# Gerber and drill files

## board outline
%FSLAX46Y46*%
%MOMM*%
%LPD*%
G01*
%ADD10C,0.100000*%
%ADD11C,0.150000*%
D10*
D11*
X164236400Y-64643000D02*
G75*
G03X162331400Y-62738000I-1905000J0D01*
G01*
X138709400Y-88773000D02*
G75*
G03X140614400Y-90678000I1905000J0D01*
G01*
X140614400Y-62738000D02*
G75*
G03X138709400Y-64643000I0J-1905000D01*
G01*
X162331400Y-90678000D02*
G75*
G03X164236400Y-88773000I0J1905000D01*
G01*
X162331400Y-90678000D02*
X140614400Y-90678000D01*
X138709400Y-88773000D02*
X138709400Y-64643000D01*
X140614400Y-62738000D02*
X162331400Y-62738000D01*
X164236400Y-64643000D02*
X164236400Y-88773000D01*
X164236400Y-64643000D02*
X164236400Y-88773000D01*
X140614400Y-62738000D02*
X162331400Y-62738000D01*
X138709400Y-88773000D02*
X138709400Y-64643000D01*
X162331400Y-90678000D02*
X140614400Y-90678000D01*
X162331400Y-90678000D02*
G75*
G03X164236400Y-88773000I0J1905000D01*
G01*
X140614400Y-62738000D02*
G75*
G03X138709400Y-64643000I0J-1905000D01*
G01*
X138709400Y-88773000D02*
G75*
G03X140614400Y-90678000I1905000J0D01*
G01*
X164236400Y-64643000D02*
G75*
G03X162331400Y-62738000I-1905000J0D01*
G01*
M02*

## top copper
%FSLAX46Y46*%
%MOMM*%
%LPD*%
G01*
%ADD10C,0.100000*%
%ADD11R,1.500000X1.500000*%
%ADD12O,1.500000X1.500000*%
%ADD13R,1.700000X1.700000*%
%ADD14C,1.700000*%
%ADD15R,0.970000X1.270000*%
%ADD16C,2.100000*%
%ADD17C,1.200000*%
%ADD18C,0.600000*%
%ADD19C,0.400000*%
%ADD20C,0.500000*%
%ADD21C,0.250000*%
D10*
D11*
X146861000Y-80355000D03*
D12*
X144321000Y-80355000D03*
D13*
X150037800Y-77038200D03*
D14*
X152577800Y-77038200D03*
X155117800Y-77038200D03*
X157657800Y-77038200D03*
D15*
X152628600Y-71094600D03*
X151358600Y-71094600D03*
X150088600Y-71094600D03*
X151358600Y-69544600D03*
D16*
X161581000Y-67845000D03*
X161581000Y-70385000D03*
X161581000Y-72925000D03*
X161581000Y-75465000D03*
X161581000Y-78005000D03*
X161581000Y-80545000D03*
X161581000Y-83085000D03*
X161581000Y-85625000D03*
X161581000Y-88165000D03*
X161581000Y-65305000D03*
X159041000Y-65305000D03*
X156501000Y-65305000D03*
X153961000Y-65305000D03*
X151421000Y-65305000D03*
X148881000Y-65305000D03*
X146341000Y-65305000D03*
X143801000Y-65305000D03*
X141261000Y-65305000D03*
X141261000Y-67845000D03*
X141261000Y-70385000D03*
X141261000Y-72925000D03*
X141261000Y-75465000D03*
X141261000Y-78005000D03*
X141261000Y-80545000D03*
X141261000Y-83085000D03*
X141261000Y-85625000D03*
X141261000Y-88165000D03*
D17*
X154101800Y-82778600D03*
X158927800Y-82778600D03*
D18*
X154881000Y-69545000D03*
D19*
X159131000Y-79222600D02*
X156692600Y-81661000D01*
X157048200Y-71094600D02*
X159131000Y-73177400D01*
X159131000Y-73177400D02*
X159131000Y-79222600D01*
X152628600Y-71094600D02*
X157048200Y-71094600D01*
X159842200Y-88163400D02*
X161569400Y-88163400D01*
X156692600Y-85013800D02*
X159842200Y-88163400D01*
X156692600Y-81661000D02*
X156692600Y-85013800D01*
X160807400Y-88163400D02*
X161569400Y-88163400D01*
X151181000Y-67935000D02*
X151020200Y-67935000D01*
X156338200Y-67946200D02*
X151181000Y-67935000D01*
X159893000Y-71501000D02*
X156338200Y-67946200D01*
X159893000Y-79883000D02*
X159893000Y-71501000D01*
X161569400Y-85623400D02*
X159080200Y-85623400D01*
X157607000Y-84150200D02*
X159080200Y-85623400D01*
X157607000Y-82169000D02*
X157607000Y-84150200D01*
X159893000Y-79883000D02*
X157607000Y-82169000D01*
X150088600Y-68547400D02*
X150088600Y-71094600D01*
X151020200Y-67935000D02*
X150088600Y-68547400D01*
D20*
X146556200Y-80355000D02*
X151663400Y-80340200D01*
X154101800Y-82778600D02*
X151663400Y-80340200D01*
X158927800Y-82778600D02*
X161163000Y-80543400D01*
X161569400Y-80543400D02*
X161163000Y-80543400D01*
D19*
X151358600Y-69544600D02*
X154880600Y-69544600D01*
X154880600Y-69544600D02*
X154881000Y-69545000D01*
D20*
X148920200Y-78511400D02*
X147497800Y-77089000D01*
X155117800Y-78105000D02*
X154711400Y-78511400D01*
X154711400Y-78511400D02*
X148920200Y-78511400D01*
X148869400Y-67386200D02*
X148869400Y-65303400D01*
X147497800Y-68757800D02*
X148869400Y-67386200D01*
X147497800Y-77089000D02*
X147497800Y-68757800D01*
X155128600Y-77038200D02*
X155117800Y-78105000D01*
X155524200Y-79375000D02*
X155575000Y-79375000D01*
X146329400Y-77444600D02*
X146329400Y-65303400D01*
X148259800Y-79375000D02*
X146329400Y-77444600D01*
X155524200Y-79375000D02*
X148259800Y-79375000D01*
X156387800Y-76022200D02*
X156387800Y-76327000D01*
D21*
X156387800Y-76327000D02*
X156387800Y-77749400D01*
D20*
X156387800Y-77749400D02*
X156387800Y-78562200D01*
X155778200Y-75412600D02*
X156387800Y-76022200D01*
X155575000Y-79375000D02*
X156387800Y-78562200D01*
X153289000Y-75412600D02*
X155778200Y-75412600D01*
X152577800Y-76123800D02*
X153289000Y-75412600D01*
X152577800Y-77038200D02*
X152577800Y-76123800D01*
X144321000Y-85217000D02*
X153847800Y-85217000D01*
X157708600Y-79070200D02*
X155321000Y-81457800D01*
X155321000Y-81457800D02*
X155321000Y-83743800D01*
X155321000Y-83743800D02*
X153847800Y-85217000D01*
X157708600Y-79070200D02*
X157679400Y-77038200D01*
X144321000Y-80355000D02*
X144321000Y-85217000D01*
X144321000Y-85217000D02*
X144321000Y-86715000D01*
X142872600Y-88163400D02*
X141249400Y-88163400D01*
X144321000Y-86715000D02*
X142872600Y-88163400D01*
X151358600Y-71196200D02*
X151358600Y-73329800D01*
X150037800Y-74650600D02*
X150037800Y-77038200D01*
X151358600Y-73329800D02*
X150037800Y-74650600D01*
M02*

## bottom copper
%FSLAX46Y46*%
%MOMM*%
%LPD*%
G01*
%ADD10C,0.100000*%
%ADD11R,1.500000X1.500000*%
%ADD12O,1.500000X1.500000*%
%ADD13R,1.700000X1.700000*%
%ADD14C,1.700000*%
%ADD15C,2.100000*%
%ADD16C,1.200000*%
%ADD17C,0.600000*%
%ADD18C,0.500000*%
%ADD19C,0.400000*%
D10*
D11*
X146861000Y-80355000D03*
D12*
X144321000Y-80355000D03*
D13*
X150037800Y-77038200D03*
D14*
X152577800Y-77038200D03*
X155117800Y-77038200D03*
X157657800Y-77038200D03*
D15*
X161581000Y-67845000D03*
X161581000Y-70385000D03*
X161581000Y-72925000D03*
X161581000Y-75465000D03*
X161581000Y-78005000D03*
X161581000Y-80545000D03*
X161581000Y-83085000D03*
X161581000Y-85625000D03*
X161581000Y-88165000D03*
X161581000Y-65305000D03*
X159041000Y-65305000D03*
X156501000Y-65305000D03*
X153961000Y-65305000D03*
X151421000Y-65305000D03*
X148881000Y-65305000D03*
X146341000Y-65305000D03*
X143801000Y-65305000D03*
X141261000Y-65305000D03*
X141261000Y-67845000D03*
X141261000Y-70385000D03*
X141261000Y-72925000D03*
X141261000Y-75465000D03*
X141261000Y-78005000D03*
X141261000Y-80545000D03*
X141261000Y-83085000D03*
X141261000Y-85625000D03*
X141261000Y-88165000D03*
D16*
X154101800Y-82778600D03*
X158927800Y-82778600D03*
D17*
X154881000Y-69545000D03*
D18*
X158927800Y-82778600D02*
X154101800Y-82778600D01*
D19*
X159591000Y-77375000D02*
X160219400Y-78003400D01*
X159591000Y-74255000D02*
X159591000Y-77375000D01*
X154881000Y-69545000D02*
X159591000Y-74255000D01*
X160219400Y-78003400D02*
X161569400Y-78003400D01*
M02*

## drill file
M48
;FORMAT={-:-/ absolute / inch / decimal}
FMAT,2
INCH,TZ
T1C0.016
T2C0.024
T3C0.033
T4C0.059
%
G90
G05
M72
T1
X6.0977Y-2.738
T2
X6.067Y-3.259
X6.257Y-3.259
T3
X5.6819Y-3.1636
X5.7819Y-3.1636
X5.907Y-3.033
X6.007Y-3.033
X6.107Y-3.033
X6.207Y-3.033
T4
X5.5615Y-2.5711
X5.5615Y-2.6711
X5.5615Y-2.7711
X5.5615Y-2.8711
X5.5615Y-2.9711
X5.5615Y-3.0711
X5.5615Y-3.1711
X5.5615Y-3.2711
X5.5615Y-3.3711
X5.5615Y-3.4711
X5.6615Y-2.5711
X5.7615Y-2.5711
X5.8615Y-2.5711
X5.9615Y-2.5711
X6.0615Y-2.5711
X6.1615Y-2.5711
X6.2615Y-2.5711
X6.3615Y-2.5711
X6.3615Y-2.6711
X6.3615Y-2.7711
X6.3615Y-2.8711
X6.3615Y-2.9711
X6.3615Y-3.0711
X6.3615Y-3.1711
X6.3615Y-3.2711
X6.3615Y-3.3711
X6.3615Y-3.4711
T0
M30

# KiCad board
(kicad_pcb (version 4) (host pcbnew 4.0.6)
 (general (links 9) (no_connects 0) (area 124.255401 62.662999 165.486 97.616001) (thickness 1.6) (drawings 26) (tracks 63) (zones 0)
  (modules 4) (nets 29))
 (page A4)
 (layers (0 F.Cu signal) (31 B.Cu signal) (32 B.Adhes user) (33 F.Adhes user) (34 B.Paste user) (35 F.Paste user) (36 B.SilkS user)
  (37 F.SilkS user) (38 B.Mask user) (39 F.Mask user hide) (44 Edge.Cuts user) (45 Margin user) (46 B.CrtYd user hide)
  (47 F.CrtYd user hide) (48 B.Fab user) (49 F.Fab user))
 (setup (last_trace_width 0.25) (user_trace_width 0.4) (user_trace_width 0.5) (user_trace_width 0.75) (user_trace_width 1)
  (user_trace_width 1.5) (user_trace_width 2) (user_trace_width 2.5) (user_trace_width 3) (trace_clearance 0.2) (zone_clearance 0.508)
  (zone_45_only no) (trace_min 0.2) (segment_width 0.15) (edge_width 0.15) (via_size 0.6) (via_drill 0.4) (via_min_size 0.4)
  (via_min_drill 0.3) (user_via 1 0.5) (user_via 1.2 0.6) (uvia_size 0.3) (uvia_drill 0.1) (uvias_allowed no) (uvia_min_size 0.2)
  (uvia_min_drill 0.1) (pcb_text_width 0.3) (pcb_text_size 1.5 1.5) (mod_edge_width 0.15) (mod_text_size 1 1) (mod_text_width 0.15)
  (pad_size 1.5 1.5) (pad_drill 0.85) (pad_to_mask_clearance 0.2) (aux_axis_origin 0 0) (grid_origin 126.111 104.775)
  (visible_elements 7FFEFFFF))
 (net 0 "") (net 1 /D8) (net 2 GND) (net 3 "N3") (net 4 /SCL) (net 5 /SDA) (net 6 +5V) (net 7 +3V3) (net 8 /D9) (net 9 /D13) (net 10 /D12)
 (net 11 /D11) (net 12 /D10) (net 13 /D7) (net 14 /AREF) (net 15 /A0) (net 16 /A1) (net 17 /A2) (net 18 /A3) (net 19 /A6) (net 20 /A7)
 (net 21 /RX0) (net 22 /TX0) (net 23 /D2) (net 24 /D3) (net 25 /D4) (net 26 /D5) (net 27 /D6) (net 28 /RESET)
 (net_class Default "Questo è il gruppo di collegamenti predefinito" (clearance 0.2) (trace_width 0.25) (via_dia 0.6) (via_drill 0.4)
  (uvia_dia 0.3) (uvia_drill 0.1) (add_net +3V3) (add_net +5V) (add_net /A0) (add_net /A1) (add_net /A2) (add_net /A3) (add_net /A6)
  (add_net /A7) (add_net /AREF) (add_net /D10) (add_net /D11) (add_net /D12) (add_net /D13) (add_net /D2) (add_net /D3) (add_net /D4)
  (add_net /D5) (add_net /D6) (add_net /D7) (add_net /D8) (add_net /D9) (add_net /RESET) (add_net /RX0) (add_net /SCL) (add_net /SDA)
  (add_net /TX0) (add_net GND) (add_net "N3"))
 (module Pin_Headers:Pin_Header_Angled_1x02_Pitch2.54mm (layer F.Cu) (at 146.861 80.355 270)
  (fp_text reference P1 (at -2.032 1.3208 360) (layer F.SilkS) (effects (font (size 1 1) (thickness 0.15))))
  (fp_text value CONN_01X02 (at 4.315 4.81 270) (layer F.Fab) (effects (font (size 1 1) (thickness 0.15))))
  (pad 1 thru_hole rect (at 0 0 270) (size 1.5 1.5) (drill 0.85) (layers *.Cu *.Mask) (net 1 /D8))
  (pad 2 thru_hole oval (at 0 2.54 270) (size 1.5 1.5) (drill 0.85) (layers *.Cu *.Mask) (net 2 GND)))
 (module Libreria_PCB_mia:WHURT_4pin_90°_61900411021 (layer F.Cu) (at 150.0378 77.0382)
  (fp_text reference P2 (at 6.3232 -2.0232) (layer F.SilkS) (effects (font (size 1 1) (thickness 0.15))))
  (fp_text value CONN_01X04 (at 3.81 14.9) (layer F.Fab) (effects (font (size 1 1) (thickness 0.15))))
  (pad 1 thru_hole rect (at 0 0) (size 1.7 1.7) (drill 0.85) (layers *.Cu *.Mask) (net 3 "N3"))
  (pad 2 thru_hole circle (at 2.54 0) (size 1.7 1.7) (drill 0.85) (layers *.Cu *.Mask) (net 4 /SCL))
  (pad 3 thru_hole circle (at 5.08 0) (size 1.7 1.7) (drill 0.85) (layers *.Cu *.Mask) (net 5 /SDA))
  (pad 4 thru_hole circle (at 7.62 0) (size 1.7 1.7) (drill 0.85) (layers *.Cu *.Mask) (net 2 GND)))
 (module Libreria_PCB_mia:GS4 (layer F.Cu) (at 151.3586 71.0946 270)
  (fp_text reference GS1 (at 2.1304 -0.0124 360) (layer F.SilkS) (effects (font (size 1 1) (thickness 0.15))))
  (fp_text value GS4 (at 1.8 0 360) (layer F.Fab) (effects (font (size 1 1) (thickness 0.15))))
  (pad 1 smd rect (at 0 -1.27 270) (size 1.27 0.97) (layers F.Cu F.Paste F.Mask) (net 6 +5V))
  (pad 2 smd rect (at 0 0 270) (size 1.27 0.97) (layers F.Cu F.Paste F.Mask) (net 3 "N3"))
  (pad 3 smd rect (at 0 1.27 270) (size 1.27 0.97) (layers F.Cu F.Paste F.Mask) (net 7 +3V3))
  (pad 4 smd rect (at -1.55 0 270) (size 1.27 0.97) (layers F.Cu F.Paste F.Mask) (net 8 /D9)))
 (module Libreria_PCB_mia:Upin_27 (layer B.Cu) (at 161.581 88.165 180)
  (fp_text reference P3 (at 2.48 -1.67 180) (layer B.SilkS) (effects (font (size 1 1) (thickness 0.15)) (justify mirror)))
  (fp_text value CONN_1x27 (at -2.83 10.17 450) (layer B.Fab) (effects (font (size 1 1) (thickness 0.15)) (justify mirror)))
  (pad 9 thru_hole circle (at 0 20.32 180) (size 2.1 2.1) (drill 1.5) (layers *.Cu *.Mask) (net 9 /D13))
  (pad 8 thru_hole circle (at 0 17.78 180) (size 2.1 2.1) (drill 1.5) (layers *.Cu *.Mask) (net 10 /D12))
  (pad 7 thru_hole circle (at 0 15.24 180) (size 2.1 2.1) (drill 1.5) (layers *.Cu *.Mask) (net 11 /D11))
  (pad 6 thru_hole circle (at 0 12.7 180) (size 2.1 2.1) (drill 1.5) (layers *.Cu *.Mask) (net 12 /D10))
  (pad 5 thru_hole circle (at 0 10.16 180) (size 2.1 2.1) (drill 1.5) (layers *.Cu *.Mask) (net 8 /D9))
  (pad 4 thru_hole circle (at 0 7.62 180) (size 2.1 2.1) (drill 1.5) (layers *.Cu *.Mask) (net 1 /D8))
  (pad 3 thru_hole circle (at 0 5.08 180) (size 2.1 2.1) (drill 1.5) (layers *.Cu *.Mask) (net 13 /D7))
  (pad 2 thru_hole circle (at 0 2.54 180) (size 2.1 2.1) (drill 1.5) (layers *.Cu *.Mask) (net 7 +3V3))
  (pad 1 thru_hole circle (at 0 0 180) (size 2.1 2.1) (drill 1.5) (layers *.Cu *.Mask) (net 6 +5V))
  (pad 10 thru_hole circle (at 0 22.86 180) (size 2.1 2.1) (drill 1.5) (layers *.Cu *.Mask) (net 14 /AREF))
  (pad 11 thru_hole circle (at 2.54 22.86 180) (size 2.1 2.1) (drill 1.5) (layers *.Cu *.Mask) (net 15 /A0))
  (pad 12 thru_hole circle (at 5.08 22.86 180) (size 2.1 2.1) (drill 1.5) (layers *.Cu *.Mask) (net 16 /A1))
  (pad 13 thru_hole circle (at 7.62 22.86 180) (size 2.1 2.1) (drill 1.5) (layers *.Cu *.Mask) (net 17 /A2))
  (pad 14 thru_hole circle (at 10.16 22.86 180) (size 2.1 2.1) (drill 1.5) (layers *.Cu *.Mask) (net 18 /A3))
  (pad 15 thru_hole circle (at 12.7 22.86 180) (size 2.1 2.1) (drill 1.5) (layers *.Cu *.Mask) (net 5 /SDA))
  (pad 16 thru_hole circle (at 15.24 22.86 180) (size 2.1 2.1) (drill 1.5) (layers *.Cu *.Mask) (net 4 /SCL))
  (pad 17 thru_hole circle (at 17.78 22.86 180) (size 2.1 2.1) (drill 1.5) (layers *.Cu *.Mask) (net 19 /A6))
  (pad 18 thru_hole circle (at 20.32 22.86 180) (size 2.1 2.1) (drill 1.5) (layers *.Cu *.Mask) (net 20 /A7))
  (pad 19 thru_hole circle (at 20.32 20.32 180) (size 2.1 2.1) (drill 1.5) (layers *.Cu *.Mask) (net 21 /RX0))
  (pad 20 thru_hole circle (at 20.32 17.78 180) (size 2.1 2.1) (drill 1.5) (layers *.Cu *.Mask) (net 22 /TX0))
  (pad 21 thru_hole circle (at 20.32 15.24 180) (size 2.1 2.1) (drill 1.5) (layers *.Cu *.Mask) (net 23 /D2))
  (pad 22 thru_hole circle (at 20.32 12.7 180) (size 2.1 2.1) (drill 1.5) (layers *.Cu *.Mask) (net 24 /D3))
  (pad 23 thru_hole circle (at 20.32 10.16 180) (size 2.1 2.1) (drill 1.5) (layers *.Cu *.Mask) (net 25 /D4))
  (pad 24 thru_hole circle (at 20.32 7.62 180) (size 2.1 2.1) (drill 1.5) (layers *.Cu *.Mask) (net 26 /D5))
  (pad 25 thru_hole circle (at 20.32 5.08 180) (size 2.1 2.1) (drill 1.5) (layers *.Cu *.Mask) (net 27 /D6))
  (pad 26 thru_hole circle (at 20.32 2.54 180) (size 2.1 2.1) (drill 1.5) (layers *.Cu *.Mask) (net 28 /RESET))
  (pad 27 thru_hole circle (at 20.32 0 180) (size 2.1 2.1) (drill 1.5) (layers *.Cu *.Mask) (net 2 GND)))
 (gr_arc (start 162.3314 64.643) (end 162.3314 62.738) (angle 90) (layer Edge.Cuts) (width 0.15))
 (gr_arc (start 140.6144 88.773) (end 140.6144 90.678) (angle 90) (layer Edge.Cuts) (width 0.15))
 (gr_arc (start 140.6144 64.643) (end 138.7094 64.643) (angle 90) (layer Edge.Cuts) (width 0.15))
 (gr_arc (start 162.3314 88.773) (end 164.2364 88.773) (angle 90) (layer Edge.Cuts) (width 0.15))
 (gr_line (start 162.3314 90.678) (end 140.6144 90.678) (angle 90) (layer Edge.Cuts) (width 0.15))
 (gr_line (start 138.7094 88.773) (end 138.7094 64.643) (angle 90) (layer Edge.Cuts) (width 0.15))
 (gr_line (start 140.6144 62.738) (end 162.3314 62.738) (angle 90) (layer Edge.Cuts) (width 0.15))
 (gr_line (start 164.2364 64.643) (end 164.2364 88.773) (angle 90) (layer Edge.Cuts) (width 0.15))
 (gr_line (start 164.2364 64.643) (end 164.2364 88.773) (angle 90) (layer Edge.Cuts) (width 0.15))
 (gr_line (start 140.6144 62.738) (end 162.3314 62.738) (angle 90) (layer Edge.Cuts) (width 0.15))
 (gr_line (start 138.7094 88.773) (end 138.7094 64.643) (angle 90) (layer Edge.Cuts) (width 0.15))
 (gr_line (start 162.3314 90.678) (end 140.6144 90.678) (angle 90) (layer Edge.Cuts) (width 0.15))
 (gr_arc (start 162.3314 88.773) (end 164.2364 88.773) (angle 90) (layer Edge.Cuts) (width 0.15))
 (gr_arc (start 140.6144 64.643) (end 138.7094 64.643) (angle 90) (layer Edge.Cuts) (width 0.15))
 (gr_arc (start 140.6144 88.773) (end 140.6144 90.678) (angle 90) (layer Edge.Cuts) (width 0.15))
 (gr_arc (start 162.3314 64.643) (end 162.3314 62.738) (angle 90) (layer Edge.Cuts) (width 0.15))
 (segment (start 159.131 79.2226) (end 156.6926 81.661) (width 0.4) (layer F.Cu) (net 6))
 (segment (start 157.0482 71.0946) (end 159.131 73.1774) (width 0.4) (layer F.Cu) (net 6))
 (segment (start 159.131 73.1774) (end 159.131 79.2226) (width 0.4) (layer F.Cu) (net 6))
 (segment (start 152.6286 71.0946) (end 157.0482 71.0946) (width 0.4) (layer F.Cu) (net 6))
 (segment (start 159.8422 88.1634) (end 161.5694 88.1634) (width 0.4) (layer F.Cu) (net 6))
 (segment (start 156.6926 85.0138) (end 159.8422 88.1634) (width 0.4) (layer F.Cu) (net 6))
 (segment (start 156.6926 81.661) (end 156.6926 85.0138) (width 0.4) (layer F.Cu) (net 6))
 (segment (start 160.8074 88.1634) (end 161.5694 88.1634) (width 0.4) (layer F.Cu) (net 6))
 (segment (start 151.181 67.935) (end 151.0202 67.935) (width 0.4) (layer F.Cu) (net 7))
 (segment (start 156.3382 67.9462) (end 151.181 67.935) (width 0.4) (layer F.Cu) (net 7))
 (segment (start 159.893 71.501) (end 156.3382 67.9462) (width 0.4) (layer F.Cu) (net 7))
 (segment (start 159.893 79.883) (end 159.893 71.501) (width 0.4) (layer F.Cu) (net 7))
 (segment (start 161.5694 85.6234) (end 159.0802 85.6234) (width 0.4) (layer F.Cu) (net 7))
 (segment (start 157.607 84.1502) (end 159.0802 85.6234) (width 0.4) (layer F.Cu) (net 7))
 (segment (start 157.607 82.169) (end 157.607 84.1502) (width 0.4) (layer F.Cu) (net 7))
 (segment (start 159.893 79.883) (end 157.607 82.169) (width 0.4) (layer F.Cu) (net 7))
 (segment (start 150.0886 68.5474) (end 150.0886 71.0946) (width 0.4) (layer F.Cu) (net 7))
 (segment (start 151.0202 67.935) (end 150.0886 68.5474) (width 0.4) (layer F.Cu) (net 7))
 (segment (start 146.5562 80.355) (end 151.6634 80.3402) (width 0.5) (layer F.Cu) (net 1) (status 10))
 (segment (start 158.9278 82.7786) (end 154.1018 82.7786) (width 0.5) (layer B.Cu) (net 1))
 (segment (start 154.1018 82.7786) (end 151.6634 80.3402) (width 0.5) (layer F.Cu) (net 1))
 (via (at 154.1018 82.7786) (size 1.2) (drill 0.6) (layers F.Cu B.Cu) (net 1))
 (via (at 158.9278 82.7786) (size 1.2) (drill 0.6) (layers F.Cu B.Cu) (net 1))
 (segment (start 158.9278 82.7786) (end 161.163 80.5434) (width 0.5) (layer F.Cu) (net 1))
 (segment (start 161.5694 80.5434) (end 161.163 80.5434) (width 0.5) (layer F.Cu) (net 1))
 (segment (start 151.3586 69.5446) (end 154.8806 69.5446) (width 0.4) (layer F.Cu) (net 8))
 (via (at 154.881 69.545) (size 0.6) (drill 0.4) (layers F.Cu B.Cu) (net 8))
 (segment (start 154.8806 69.5446) (end 154.881 69.545) (width 0.4) (layer F.Cu) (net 8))
 (segment (start 159.591 77.375) (end 160.2194 78.0034) (width 0.4) (layer B.Cu) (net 8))
 (segment (start 159.591 74.255) (end 159.591 77.375) (width 0.4) (layer B.Cu) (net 8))
 (segment (start 154.881 69.545) (end 159.591 74.255) (width 0.4) (layer B.Cu) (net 8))
 (segment (start 160.2194 78.0034) (end 161.5694 78.0034) (width 0.4) (layer B.Cu) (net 8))
 (segment (start 148.9202 78.5114) (end 147.4978 77.089) (width 0.5) (layer F.Cu) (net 5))
 (segment (start 155.1178 78.105) (end 154.7114 78.5114) (width 0.5) (layer F.Cu) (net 5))
 (segment (start 154.7114 78.5114) (end 148.9202 78.5114) (width 0.5) (layer F.Cu) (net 5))
 (segment (start 148.8694 67.3862) (end 148.8694 65.3034) (width 0.5) (layer F.Cu) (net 5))
 (segment (start 147.4978 68.7578) (end 148.8694 67.3862) (width 0.5) (layer F.Cu) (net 5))
 (segment (start 147.4978 77.089) (end 147.4978 68.7578) (width 0.5) (layer F.Cu) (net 5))
 (segment (start 155.1286 77.0382) (end 155.1178 78.105) (width 0.5) (layer F.Cu) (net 5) (status 10))
 (segment (start 155.5242 79.375) (end 155.575 79.375) (width 0.5) (layer F.Cu) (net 4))
 (segment (start 146.3294 77.4446) (end 146.3294 65.3034) (width 0.5) (layer F.Cu) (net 4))
 (segment (start 148.2598 79.375) (end 146.3294 77.4446) (width 0.5) (layer F.Cu) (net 4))
 (segment (start 155.5242 79.375) (end 148.2598 79.375) (width 0.5) (layer F.Cu) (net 4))
 (segment (start 156.3878 76.0222) (end 156.3878 76.327) (width 0.5) (layer F.Cu) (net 4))
 (segment (start 156.3878 76.327) (end 156.3878 77.7494) (width 0.25) (layer F.Cu) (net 4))
 (segment (start 156.3878 77.7494) (end 156.3878 78.5622) (width 0.5) (layer F.Cu) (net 4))
 (segment (start 155.7782 75.4126) (end 156.3878 76.0222) (width 0.5) (layer F.Cu) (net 4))
 (segment (start 155.575 79.375) (end 156.3878 78.5622) (width 0.5) (layer F.Cu) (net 4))
 (segment (start 153.289 75.4126) (end 155.7782 75.4126) (width 0.5) (layer F.Cu) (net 4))
 (segment (start 152.5778 76.1238) (end 153.289 75.4126) (width 0.5) (layer F.Cu) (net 4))
 (segment (start 152.5778 77.0382) (end 152.5778 76.1238) (width 0.5) (layer F.Cu) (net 4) (status 10))
 (segment (start 144.321 85.217) (end 153.8478 85.217) (width 0.5) (layer F.Cu) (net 2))
 (segment (start 157.7086 79.0702) (end 155.321 81.4578) (width 0.5) (layer F.Cu) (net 2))
 (segment (start 155.321 81.4578) (end 155.321 83.7438) (width 0.5) (layer F.Cu) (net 2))
 (segment (start 155.321 83.7438) (end 153.8478 85.217) (width 0.5) (layer F.Cu) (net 2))
 (segment (start 157.7086 79.0702) (end 157.6794 77.0382) (width 0.5) (layer F.Cu) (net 2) (status 10))
 (segment (start 144.321 80.355) (end 144.321 85.217) (width 0.5) (layer F.Cu) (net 2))
 (segment (start 144.321 85.217) (end 144.321 86.715) (width 0.5) (layer F.Cu) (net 2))
 (segment (start 142.8726 88.1634) (end 141.2494 88.1634) (width 0.5) (layer F.Cu) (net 2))
 (segment (start 144.321 86.715) (end 142.8726 88.1634) (width 0.5) (layer F.Cu) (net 2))
 (segment (start 151.3586 71.1962) (end 151.3586 73.3298) (width 0.5) (layer F.Cu) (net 3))
 (segment (start 150.0378 74.6506) (end 150.0378 77.0382) (width 0.5) (layer F.Cu) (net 3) (status 20))
 (segment (start 151.3586 73.3298) (end 150.0378 74.6506) (width 0.5) (layer F.Cu) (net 3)))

